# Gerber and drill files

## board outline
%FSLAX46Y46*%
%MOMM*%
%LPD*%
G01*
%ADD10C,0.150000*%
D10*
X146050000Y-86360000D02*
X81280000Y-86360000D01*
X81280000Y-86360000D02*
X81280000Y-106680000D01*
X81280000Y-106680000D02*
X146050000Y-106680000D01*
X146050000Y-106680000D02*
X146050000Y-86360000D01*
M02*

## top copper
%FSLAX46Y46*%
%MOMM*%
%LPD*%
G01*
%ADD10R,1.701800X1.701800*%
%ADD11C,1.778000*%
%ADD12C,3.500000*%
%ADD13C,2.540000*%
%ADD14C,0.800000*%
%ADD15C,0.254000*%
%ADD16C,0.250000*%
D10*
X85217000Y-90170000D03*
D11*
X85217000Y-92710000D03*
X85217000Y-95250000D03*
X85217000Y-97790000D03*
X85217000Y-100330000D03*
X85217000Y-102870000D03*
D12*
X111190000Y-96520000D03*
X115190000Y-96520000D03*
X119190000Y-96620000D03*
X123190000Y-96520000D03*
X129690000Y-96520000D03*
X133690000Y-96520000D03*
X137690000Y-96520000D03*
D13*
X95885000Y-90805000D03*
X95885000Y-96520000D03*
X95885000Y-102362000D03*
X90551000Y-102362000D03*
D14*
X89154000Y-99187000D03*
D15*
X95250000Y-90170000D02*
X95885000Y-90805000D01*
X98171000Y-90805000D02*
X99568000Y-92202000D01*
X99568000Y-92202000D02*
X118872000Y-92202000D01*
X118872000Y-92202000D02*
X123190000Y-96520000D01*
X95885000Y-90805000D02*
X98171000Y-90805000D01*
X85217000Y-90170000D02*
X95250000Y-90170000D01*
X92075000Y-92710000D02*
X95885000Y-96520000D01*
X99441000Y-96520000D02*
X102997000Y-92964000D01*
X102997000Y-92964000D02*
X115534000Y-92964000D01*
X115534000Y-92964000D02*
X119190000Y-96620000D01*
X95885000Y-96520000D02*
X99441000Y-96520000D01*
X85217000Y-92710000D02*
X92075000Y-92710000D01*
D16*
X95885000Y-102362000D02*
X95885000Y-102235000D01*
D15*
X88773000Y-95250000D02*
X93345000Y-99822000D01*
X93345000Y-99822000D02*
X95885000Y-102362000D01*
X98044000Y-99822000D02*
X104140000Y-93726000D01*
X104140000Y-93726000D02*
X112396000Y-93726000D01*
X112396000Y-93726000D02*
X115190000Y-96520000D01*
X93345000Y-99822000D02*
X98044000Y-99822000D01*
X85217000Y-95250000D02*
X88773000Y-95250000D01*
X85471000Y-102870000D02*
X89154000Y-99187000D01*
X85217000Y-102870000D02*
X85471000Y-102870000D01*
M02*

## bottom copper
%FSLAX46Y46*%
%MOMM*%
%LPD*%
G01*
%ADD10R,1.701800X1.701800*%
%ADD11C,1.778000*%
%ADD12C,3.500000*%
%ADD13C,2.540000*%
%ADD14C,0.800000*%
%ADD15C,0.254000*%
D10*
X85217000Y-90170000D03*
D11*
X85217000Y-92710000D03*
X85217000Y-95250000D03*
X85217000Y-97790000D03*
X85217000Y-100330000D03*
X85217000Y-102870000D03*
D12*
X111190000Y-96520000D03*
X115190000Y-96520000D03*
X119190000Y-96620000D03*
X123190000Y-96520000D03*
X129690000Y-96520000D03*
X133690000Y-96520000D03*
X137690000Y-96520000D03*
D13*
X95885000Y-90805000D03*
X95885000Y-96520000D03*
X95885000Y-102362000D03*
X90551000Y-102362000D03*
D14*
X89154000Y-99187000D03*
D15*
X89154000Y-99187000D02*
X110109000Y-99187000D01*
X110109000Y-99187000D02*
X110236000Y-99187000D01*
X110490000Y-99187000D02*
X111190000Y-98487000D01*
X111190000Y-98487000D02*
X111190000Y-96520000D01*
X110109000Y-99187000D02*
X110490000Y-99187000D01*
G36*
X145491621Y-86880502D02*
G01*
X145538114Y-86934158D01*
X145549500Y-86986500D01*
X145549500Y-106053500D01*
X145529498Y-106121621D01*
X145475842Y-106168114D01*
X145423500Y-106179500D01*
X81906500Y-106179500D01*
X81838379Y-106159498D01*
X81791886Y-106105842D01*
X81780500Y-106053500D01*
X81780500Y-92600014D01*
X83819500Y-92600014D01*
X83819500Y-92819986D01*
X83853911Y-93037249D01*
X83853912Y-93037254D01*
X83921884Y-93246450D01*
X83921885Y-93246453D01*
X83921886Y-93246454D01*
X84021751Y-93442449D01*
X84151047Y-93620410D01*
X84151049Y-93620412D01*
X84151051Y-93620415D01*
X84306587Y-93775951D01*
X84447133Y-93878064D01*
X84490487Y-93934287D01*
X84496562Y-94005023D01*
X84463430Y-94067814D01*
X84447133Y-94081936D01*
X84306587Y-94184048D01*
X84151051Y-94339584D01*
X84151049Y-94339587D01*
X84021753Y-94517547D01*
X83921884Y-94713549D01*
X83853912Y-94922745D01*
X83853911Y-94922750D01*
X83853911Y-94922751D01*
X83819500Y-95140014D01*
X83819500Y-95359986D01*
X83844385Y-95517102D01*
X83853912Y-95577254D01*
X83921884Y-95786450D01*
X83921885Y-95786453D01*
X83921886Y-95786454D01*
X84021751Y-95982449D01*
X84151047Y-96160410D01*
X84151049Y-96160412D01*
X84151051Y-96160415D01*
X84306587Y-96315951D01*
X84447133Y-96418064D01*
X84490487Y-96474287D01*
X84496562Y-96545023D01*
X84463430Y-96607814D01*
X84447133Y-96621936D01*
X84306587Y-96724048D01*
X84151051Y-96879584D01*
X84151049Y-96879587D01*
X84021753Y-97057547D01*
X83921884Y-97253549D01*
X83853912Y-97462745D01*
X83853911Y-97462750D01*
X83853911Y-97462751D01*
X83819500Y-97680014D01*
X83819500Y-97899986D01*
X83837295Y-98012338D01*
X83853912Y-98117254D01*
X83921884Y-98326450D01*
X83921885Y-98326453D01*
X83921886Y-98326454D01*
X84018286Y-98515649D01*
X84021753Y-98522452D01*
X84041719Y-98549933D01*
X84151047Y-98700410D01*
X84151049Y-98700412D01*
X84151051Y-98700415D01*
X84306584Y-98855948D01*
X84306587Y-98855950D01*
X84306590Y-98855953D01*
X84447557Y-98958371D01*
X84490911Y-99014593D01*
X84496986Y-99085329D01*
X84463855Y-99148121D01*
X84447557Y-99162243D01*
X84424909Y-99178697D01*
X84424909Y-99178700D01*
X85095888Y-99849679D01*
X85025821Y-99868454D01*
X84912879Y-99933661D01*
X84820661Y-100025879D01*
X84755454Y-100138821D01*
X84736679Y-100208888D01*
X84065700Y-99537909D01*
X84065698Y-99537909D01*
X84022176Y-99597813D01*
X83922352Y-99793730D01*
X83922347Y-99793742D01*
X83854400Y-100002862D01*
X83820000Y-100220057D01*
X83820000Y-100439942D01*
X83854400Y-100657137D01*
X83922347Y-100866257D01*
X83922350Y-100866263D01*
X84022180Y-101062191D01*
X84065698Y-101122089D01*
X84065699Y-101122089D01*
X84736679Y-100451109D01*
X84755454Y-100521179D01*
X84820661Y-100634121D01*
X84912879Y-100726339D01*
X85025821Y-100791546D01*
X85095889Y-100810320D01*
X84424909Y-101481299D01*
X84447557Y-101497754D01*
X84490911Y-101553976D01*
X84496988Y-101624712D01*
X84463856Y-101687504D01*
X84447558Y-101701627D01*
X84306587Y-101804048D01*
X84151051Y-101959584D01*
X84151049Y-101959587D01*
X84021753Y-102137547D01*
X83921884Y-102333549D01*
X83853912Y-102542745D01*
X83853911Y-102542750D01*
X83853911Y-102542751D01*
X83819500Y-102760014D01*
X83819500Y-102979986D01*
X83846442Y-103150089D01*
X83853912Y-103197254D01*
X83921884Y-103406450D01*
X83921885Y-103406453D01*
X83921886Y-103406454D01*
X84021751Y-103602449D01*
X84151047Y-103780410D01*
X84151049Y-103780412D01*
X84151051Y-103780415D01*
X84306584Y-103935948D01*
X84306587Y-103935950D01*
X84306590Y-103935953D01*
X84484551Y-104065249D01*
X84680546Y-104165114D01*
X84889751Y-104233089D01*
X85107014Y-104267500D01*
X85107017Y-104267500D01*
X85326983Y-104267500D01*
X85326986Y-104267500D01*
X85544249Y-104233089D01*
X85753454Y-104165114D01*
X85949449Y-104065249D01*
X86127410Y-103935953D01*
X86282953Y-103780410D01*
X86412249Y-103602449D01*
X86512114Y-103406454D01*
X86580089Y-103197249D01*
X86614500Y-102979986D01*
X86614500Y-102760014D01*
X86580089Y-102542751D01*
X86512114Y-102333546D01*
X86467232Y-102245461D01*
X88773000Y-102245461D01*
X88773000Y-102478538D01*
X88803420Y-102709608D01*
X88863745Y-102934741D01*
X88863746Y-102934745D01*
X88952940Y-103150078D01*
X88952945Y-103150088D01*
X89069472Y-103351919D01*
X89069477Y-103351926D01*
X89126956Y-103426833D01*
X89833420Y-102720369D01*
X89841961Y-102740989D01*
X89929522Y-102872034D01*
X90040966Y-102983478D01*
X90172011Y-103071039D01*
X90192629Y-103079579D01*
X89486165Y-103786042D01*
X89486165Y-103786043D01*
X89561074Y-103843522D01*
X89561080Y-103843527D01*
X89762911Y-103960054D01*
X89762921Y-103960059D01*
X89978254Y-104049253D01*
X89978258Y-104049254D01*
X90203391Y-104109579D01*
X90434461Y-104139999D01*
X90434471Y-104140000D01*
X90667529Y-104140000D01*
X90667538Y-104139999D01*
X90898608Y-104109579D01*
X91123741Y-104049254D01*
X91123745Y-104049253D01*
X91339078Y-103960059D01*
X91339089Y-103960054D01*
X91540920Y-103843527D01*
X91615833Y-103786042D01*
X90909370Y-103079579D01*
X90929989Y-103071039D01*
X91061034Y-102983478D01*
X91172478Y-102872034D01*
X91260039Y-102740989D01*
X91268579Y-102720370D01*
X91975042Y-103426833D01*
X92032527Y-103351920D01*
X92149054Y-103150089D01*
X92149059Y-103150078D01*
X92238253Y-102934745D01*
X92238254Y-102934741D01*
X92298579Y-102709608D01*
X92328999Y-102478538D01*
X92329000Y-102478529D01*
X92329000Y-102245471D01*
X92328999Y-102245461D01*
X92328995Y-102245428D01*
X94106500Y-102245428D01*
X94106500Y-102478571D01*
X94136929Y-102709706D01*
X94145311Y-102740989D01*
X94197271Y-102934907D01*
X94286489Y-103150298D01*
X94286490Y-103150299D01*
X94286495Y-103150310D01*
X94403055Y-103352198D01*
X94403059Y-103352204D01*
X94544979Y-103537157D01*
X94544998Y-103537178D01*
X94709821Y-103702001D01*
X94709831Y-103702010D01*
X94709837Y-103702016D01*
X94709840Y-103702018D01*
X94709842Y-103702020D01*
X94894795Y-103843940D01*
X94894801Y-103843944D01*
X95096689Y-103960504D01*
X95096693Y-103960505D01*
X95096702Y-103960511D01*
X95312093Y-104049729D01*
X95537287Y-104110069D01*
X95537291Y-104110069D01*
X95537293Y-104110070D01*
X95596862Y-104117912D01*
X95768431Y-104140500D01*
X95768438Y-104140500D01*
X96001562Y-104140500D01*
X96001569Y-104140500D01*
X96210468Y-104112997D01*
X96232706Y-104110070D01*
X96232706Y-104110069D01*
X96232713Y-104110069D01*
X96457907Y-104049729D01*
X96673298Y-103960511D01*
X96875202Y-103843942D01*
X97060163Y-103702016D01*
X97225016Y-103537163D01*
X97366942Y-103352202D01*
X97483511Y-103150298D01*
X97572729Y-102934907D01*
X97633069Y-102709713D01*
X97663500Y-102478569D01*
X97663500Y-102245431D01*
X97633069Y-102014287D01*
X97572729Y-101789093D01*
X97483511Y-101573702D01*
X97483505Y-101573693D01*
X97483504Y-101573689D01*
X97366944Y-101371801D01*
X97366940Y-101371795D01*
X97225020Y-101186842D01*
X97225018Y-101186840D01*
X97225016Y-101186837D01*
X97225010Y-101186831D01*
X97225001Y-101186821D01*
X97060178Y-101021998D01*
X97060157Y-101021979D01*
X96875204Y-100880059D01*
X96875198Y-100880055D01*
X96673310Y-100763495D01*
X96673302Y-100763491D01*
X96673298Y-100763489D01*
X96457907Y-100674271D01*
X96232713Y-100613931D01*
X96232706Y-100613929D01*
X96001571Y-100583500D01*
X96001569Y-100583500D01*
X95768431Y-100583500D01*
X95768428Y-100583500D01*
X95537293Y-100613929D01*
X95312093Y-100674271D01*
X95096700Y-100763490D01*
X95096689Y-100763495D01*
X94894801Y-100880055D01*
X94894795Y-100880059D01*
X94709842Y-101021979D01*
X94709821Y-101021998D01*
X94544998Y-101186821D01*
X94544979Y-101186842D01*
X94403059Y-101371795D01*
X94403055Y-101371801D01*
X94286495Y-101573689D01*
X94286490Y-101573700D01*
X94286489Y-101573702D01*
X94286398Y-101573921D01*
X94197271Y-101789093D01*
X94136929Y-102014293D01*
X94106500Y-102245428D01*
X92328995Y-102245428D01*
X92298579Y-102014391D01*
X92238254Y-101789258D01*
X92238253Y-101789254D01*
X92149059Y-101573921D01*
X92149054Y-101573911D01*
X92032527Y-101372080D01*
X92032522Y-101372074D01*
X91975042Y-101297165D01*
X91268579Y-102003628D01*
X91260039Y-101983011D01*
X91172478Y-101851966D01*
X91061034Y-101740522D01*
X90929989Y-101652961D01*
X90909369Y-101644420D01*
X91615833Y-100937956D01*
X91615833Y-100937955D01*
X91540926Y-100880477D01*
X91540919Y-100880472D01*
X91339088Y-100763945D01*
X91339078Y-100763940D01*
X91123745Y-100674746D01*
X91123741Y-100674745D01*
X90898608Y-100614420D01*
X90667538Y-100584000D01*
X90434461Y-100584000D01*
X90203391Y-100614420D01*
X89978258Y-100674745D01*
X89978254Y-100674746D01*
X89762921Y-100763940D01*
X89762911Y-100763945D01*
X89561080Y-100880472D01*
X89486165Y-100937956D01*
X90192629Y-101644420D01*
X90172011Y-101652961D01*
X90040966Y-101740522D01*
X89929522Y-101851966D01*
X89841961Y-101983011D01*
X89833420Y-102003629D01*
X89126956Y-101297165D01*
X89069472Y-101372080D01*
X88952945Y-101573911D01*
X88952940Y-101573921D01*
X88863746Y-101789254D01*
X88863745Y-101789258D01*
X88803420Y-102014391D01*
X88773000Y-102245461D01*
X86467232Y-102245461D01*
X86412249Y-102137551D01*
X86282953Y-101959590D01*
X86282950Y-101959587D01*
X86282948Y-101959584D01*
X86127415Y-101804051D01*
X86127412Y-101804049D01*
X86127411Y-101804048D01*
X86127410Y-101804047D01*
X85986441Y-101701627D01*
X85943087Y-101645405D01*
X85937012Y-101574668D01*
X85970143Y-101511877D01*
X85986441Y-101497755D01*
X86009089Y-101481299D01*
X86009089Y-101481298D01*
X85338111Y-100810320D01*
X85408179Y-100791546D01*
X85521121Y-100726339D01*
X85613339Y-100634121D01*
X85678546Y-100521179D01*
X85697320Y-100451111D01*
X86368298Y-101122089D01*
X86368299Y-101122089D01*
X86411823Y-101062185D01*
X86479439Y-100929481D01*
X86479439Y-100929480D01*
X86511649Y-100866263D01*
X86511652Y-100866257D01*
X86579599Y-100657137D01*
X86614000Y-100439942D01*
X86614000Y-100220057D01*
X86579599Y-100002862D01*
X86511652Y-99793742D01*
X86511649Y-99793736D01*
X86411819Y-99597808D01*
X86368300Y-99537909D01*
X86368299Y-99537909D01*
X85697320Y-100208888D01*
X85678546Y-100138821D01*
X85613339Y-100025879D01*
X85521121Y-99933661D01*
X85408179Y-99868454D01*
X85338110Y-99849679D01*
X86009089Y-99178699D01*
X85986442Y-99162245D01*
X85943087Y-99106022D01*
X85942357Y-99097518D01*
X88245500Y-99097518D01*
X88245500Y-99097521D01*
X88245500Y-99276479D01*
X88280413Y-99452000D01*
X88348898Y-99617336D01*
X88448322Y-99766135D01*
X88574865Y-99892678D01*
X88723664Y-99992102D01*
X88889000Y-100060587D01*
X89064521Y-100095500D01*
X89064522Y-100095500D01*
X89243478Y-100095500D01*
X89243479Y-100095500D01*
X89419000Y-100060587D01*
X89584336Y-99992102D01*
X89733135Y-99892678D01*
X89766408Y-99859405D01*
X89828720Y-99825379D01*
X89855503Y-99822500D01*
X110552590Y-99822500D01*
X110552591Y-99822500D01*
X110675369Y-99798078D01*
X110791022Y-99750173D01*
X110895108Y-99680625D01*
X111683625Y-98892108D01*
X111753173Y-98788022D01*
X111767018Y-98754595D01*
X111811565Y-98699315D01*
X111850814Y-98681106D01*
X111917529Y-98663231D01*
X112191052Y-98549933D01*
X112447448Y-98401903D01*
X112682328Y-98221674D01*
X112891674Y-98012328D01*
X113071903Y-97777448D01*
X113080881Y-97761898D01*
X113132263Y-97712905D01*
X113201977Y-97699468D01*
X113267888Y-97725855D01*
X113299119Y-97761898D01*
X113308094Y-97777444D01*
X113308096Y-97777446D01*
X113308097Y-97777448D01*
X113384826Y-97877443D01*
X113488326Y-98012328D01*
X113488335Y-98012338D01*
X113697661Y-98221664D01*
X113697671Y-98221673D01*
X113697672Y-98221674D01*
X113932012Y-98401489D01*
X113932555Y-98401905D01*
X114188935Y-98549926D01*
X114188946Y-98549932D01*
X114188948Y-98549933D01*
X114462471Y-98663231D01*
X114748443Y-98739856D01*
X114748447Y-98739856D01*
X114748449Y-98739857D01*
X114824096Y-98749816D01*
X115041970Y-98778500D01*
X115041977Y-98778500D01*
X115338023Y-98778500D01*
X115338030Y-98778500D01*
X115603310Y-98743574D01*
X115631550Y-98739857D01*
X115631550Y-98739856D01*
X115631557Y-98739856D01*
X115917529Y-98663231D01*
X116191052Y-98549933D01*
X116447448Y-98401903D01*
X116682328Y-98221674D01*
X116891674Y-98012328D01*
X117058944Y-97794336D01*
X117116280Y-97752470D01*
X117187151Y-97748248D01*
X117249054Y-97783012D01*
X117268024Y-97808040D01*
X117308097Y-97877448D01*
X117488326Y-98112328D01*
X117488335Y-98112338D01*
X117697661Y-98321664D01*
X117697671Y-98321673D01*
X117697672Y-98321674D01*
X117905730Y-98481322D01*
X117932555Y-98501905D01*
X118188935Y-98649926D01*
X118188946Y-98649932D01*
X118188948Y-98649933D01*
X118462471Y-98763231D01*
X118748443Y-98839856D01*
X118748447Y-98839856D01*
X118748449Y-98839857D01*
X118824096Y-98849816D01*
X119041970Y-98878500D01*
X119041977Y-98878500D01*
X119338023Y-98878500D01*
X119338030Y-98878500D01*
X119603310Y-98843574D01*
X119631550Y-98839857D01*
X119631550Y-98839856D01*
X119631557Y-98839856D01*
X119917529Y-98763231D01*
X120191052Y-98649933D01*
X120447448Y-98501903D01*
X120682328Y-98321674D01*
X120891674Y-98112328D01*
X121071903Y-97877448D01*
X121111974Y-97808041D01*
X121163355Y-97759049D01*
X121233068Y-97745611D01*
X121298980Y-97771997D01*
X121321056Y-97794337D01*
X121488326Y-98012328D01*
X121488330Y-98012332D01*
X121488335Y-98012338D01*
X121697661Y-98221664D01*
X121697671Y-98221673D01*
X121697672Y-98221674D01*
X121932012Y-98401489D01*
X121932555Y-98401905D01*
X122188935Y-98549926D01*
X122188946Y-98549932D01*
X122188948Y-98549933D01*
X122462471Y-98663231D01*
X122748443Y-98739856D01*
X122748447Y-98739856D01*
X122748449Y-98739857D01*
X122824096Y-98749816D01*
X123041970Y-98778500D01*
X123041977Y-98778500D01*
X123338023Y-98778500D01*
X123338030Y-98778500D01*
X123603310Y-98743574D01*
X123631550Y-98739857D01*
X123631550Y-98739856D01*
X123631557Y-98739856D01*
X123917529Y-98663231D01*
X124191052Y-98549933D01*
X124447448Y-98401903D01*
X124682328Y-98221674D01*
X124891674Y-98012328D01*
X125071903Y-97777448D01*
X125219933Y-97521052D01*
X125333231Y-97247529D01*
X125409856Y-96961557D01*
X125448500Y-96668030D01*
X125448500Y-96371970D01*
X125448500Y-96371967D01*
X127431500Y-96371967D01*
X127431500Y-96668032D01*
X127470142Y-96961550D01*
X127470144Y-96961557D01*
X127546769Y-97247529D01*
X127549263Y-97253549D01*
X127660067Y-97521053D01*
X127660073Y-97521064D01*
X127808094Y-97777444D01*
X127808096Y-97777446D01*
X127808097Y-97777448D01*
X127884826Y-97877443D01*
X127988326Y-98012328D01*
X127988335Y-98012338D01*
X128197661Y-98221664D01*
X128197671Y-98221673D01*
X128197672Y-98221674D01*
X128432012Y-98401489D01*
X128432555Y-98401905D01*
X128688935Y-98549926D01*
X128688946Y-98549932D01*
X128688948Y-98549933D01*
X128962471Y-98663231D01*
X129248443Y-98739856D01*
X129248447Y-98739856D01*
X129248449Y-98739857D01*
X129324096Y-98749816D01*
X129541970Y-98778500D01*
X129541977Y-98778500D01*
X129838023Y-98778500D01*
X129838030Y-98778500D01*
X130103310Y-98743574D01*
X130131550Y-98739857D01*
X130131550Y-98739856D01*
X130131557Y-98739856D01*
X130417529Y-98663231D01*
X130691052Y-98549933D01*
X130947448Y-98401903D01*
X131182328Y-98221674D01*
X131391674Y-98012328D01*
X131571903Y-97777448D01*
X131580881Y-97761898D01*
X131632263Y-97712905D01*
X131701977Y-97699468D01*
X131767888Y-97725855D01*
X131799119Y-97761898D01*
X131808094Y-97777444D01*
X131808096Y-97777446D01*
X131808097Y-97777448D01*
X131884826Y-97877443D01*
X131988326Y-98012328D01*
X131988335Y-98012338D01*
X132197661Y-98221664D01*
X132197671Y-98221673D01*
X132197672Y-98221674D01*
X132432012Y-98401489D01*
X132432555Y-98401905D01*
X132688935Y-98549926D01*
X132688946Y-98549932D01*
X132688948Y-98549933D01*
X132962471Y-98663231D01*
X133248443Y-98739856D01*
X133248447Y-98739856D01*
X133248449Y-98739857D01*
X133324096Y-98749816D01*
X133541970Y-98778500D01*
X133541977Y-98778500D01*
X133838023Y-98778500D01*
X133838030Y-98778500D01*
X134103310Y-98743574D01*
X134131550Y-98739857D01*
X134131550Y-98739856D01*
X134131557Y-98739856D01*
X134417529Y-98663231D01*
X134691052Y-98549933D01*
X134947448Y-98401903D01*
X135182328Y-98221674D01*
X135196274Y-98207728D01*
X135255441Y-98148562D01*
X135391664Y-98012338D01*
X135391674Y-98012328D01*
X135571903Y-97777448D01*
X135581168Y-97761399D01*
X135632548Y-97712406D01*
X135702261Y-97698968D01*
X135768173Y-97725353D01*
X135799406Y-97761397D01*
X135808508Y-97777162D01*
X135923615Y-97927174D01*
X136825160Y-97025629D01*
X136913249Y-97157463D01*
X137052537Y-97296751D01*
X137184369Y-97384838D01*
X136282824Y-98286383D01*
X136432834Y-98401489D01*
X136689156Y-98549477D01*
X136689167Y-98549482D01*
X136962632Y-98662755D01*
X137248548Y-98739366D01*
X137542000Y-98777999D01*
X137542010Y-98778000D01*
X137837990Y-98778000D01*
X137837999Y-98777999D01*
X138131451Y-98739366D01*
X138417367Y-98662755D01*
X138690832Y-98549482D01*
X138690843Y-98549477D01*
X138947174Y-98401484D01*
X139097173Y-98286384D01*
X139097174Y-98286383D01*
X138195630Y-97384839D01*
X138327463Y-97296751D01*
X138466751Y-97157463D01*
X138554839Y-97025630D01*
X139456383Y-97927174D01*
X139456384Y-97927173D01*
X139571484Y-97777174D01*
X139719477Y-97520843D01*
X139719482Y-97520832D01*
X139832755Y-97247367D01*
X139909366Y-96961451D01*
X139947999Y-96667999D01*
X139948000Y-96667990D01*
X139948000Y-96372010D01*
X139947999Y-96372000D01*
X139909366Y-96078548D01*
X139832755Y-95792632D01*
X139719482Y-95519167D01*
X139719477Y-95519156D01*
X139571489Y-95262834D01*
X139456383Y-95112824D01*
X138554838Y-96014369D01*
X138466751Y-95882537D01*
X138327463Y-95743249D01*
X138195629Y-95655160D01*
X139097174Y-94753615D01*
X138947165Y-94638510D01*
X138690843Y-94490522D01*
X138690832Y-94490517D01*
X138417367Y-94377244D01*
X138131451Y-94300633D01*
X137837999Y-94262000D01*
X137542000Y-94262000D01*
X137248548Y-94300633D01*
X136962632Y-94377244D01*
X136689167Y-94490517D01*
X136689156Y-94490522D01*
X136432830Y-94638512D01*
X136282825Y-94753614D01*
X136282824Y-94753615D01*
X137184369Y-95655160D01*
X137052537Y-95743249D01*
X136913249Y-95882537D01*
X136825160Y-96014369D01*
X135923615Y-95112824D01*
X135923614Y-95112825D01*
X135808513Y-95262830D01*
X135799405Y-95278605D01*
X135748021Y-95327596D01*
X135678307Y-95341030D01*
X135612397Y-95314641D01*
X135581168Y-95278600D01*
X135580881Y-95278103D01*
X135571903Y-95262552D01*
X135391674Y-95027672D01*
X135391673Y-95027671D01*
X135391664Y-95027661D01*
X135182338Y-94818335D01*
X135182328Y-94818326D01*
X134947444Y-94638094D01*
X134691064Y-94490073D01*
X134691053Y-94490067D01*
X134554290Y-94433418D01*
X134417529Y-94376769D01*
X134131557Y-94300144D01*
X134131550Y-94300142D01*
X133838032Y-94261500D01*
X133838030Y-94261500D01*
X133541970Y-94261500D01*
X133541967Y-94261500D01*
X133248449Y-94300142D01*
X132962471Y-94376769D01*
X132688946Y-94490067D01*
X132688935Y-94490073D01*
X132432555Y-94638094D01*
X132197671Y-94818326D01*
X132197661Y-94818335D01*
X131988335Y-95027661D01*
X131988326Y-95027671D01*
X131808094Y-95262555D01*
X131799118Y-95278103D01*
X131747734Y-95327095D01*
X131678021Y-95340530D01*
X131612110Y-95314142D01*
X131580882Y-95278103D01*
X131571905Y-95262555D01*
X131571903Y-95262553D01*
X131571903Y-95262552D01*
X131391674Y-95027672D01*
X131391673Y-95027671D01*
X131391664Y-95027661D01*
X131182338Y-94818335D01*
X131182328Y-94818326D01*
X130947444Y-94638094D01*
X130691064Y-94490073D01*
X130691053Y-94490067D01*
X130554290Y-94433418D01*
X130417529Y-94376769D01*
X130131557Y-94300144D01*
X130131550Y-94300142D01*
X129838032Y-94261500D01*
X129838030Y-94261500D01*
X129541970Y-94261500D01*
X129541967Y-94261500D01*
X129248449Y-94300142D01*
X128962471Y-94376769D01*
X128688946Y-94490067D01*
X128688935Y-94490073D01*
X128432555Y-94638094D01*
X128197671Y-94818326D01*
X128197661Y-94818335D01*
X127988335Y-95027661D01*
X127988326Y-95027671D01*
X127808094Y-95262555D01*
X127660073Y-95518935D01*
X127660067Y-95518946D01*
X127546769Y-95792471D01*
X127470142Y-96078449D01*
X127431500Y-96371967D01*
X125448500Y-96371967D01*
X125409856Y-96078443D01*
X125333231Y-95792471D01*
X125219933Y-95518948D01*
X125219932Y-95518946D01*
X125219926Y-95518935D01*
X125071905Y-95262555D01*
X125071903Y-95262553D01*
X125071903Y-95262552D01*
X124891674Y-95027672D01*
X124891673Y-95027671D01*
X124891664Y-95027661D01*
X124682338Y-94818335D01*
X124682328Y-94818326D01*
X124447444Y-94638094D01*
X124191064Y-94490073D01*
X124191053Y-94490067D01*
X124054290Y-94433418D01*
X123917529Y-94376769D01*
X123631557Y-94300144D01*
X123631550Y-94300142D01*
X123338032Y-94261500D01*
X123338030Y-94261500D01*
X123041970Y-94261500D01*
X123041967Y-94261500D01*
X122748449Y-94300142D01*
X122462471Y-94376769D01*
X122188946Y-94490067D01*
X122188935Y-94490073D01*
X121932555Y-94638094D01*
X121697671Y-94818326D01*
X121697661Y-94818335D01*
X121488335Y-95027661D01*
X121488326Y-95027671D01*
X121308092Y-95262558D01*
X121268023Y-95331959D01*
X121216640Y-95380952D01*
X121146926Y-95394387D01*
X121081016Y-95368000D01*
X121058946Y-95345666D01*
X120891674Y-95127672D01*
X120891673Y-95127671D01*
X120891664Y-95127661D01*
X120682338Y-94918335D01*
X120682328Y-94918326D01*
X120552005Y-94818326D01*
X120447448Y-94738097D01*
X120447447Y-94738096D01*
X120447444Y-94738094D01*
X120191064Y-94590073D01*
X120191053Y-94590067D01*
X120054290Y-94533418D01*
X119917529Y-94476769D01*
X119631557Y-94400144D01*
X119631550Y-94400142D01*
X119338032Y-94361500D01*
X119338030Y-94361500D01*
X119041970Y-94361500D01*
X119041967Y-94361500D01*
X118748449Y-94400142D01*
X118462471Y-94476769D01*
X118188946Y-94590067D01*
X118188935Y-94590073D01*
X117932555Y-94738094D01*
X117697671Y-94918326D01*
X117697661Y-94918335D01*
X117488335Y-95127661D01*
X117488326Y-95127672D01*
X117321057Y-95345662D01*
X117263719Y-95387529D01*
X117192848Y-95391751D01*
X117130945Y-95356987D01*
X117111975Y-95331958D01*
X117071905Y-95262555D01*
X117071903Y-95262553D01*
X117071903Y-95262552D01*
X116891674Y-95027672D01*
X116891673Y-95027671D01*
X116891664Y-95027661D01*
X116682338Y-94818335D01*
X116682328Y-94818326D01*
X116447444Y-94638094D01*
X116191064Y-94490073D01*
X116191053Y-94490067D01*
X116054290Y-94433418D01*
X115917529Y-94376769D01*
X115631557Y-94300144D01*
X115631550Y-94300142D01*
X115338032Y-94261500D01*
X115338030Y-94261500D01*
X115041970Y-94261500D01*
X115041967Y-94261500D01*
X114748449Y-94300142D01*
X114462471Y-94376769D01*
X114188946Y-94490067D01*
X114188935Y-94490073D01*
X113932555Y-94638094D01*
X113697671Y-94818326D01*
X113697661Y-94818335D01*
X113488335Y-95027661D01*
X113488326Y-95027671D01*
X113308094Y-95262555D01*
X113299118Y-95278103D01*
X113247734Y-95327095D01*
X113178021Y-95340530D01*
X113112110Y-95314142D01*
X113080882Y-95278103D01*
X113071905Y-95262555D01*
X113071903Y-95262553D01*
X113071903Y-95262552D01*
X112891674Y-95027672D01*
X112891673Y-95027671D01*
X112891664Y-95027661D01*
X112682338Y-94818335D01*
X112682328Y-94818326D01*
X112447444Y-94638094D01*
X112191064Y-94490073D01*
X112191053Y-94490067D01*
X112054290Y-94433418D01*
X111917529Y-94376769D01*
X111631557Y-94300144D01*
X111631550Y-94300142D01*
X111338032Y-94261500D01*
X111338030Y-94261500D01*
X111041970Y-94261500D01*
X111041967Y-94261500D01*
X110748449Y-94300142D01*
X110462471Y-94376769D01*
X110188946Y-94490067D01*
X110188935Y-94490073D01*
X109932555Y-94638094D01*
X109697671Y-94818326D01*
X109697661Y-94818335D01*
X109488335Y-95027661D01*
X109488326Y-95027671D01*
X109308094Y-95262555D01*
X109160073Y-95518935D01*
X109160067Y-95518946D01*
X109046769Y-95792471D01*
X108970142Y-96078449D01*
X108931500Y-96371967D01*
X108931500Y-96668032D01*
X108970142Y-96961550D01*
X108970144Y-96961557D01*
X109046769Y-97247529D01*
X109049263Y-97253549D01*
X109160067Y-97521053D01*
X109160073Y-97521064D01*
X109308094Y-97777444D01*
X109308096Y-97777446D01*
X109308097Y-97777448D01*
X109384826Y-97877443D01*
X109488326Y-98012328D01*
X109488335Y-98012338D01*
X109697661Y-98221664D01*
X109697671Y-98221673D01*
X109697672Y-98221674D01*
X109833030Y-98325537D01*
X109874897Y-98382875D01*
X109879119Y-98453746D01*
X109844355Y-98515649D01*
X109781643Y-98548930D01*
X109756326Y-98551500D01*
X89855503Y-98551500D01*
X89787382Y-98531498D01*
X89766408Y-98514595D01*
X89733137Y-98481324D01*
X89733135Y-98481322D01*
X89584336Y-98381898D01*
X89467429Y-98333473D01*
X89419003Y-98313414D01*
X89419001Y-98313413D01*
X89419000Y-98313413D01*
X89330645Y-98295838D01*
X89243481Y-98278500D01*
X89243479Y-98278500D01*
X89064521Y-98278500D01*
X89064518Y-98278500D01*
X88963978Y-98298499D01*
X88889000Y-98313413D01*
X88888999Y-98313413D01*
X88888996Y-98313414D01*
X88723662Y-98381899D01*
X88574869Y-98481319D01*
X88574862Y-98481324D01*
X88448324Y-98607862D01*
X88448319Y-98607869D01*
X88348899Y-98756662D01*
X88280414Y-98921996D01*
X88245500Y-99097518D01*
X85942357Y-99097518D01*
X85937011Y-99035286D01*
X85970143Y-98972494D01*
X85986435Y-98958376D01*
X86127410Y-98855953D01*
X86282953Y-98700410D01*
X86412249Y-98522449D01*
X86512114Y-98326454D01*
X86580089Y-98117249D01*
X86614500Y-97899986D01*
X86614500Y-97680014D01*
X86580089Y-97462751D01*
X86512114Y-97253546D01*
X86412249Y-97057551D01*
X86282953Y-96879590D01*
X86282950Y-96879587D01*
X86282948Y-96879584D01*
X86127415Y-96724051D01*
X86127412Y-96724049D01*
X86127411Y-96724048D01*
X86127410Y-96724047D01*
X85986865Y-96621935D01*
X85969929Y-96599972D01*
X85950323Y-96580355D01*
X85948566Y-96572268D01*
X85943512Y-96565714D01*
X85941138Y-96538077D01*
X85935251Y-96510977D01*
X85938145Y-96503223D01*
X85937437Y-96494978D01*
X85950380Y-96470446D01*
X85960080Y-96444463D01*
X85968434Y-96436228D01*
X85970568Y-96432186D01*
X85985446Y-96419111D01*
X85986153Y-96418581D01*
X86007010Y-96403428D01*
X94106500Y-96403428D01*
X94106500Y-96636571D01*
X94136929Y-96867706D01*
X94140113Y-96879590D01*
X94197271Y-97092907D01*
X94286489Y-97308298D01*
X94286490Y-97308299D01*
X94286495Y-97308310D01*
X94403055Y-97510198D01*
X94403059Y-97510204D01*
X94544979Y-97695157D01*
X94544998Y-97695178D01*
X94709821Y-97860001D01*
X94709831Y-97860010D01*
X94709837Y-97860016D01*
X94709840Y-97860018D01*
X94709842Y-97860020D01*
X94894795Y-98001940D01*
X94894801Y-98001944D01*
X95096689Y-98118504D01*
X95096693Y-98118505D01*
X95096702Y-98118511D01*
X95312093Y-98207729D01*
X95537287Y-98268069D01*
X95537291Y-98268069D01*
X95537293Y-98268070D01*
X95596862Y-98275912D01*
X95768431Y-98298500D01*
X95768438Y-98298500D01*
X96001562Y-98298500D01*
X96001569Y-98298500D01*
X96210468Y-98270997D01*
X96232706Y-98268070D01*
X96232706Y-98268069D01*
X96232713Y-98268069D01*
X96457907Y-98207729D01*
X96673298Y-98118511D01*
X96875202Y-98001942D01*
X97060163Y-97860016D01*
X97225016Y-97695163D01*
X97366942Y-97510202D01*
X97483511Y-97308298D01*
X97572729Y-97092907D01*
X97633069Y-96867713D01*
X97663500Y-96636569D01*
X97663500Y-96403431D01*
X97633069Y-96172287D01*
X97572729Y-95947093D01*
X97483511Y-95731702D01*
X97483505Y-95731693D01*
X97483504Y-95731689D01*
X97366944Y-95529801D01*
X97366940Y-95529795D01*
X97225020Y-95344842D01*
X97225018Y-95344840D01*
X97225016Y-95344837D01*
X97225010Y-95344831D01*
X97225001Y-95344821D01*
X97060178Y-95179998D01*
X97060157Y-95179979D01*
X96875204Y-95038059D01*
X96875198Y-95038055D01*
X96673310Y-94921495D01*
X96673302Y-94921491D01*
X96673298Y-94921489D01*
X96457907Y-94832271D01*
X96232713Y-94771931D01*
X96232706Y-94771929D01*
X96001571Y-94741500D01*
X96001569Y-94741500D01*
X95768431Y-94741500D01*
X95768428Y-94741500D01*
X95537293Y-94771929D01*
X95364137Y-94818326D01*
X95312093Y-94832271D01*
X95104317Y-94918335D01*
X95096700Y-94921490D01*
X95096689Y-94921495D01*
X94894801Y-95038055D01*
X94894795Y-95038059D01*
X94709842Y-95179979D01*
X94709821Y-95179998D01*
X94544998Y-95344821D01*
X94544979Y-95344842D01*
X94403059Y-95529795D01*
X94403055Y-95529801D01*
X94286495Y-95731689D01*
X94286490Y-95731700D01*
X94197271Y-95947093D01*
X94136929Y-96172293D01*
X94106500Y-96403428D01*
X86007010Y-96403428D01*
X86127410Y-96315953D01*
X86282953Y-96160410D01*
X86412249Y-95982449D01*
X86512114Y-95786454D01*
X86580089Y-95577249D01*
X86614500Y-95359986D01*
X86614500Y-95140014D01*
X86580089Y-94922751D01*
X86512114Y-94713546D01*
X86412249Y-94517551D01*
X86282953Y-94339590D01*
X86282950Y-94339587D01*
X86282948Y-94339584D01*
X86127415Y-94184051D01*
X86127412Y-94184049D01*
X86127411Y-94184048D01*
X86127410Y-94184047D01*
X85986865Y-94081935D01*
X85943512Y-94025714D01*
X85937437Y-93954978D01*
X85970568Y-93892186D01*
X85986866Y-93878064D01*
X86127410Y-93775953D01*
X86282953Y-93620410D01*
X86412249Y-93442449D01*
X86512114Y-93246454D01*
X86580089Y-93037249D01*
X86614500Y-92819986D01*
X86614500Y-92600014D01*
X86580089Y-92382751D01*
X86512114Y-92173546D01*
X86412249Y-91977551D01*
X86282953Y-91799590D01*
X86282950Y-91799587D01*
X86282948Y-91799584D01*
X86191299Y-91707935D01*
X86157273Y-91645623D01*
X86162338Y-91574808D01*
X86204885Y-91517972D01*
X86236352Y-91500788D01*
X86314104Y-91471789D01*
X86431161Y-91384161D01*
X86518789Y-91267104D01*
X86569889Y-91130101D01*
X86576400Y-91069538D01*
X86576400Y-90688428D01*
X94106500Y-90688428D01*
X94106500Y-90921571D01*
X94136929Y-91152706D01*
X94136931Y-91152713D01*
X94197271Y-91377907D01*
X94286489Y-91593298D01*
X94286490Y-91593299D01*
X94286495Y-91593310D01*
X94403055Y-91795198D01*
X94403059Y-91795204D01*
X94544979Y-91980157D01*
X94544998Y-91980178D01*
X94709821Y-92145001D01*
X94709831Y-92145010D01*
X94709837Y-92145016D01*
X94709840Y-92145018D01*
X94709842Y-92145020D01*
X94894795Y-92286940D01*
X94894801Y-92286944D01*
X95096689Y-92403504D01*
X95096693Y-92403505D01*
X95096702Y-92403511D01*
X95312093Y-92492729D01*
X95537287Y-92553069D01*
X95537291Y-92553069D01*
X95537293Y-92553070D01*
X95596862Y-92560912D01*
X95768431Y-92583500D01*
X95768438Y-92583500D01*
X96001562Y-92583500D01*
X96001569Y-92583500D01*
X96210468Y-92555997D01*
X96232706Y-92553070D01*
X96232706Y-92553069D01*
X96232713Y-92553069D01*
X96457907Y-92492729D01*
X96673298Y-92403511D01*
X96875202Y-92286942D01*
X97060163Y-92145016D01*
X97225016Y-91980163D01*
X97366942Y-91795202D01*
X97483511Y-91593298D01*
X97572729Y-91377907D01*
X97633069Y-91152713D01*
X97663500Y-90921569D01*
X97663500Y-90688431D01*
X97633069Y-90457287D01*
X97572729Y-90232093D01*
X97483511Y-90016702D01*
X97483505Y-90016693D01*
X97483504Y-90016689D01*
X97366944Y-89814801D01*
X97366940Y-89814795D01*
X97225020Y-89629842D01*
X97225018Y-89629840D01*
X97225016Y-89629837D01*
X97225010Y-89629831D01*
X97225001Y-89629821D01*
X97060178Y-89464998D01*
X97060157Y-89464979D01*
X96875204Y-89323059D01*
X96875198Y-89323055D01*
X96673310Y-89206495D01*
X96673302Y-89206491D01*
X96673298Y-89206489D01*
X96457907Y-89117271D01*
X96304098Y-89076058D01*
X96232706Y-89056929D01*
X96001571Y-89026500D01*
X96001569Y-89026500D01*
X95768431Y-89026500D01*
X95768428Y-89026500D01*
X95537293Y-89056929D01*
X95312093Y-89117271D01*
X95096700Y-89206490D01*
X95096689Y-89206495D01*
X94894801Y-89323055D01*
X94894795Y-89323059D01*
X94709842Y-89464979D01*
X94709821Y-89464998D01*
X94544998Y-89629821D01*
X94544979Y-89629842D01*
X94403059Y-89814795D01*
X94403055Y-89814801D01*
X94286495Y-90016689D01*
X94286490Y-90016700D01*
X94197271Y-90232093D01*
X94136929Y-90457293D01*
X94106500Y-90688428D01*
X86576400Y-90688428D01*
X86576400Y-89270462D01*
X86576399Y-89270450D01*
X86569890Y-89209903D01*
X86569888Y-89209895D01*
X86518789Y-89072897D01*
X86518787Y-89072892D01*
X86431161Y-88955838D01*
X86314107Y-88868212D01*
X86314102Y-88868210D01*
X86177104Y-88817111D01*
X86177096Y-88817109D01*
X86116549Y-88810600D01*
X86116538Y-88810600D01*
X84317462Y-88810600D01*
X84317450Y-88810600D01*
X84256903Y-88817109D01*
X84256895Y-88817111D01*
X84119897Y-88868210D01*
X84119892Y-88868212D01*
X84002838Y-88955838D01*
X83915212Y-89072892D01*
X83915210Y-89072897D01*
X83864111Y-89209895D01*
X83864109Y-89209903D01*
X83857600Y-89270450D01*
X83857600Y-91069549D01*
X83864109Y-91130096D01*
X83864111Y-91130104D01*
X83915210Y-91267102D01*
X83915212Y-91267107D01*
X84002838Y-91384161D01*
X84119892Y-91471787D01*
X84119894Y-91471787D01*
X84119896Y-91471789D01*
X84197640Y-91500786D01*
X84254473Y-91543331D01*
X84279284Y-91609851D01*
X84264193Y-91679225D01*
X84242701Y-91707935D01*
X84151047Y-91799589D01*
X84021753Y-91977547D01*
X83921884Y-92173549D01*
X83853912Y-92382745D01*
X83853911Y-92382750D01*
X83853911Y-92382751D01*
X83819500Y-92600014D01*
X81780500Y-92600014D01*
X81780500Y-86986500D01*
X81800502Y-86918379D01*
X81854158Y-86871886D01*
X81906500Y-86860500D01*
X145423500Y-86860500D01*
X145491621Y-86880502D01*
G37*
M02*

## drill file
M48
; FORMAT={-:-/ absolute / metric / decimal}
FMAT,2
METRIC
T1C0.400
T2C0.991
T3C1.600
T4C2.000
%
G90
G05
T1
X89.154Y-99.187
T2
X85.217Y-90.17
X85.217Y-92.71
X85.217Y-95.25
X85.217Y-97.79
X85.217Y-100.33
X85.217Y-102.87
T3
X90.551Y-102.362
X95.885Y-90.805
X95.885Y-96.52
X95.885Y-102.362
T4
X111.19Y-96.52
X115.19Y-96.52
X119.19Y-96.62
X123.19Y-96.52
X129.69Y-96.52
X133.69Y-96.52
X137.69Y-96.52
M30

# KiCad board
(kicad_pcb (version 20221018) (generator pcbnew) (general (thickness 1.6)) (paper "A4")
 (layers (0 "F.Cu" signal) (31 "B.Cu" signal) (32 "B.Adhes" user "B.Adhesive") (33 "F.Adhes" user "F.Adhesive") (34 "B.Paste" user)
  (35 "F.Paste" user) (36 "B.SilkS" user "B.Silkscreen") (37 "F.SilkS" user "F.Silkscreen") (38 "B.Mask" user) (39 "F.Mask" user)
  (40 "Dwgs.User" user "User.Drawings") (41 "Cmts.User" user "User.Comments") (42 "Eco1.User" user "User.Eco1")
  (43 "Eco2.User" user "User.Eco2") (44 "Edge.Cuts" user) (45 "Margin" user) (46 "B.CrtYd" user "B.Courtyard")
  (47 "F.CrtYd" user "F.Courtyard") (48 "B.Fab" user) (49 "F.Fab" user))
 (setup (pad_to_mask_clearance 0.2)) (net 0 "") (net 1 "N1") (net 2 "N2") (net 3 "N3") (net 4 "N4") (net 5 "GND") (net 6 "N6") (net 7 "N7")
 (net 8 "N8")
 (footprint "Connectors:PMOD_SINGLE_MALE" (layer "F.Cu") (at 83.185 96.52 90)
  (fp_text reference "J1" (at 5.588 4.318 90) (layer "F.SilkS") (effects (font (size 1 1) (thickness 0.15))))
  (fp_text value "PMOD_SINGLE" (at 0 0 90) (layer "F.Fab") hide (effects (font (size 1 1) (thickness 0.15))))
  (pad "1" thru_hole rect (at 6.35 2.032 270) (size 1.7018 1.7018) (drill 0.9906) (layers "*.Cu" "*.Mask" "F.SilkS") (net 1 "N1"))
  (pad "2" thru_hole circle (at 3.81 2.032 270) (size 1.778 1.778) (drill 0.9906) (layers "*.Cu" "*.Mask" "F.SilkS") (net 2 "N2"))
  (pad "3" thru_hole circle (at 1.27 2.032 270) (size 1.778 1.778) (drill 0.9906) (layers "*.Cu" "*.Mask" "F.SilkS") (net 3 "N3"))
  (pad "4" thru_hole circle (at -1.27 2.032 270) (size 1.778 1.778) (drill 0.9906) (layers "*.Cu" "*.Mask" "F.SilkS") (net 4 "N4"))
  (pad "5" thru_hole circle (at -3.81 2.032 270) (size 1.778 1.778) (drill 0.9906) (layers "*.Cu" "*.Mask" "F.SilkS") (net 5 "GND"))
  (pad "6" thru_hole circle (at -6.35 2.032 270) (size 1.778 1.778) (drill 0.9906) (layers "*.Cu" "*.Mask" "F.SilkS") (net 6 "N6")))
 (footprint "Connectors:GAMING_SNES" (layer "F.Cu") (at 123.19 96.52)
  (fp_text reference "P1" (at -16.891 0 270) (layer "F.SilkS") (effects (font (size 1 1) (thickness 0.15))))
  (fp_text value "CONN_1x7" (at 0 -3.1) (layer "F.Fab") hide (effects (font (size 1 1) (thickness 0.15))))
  (pad "1" thru_hole circle (at -12 0) (size 3.5 3.5) (drill 2) (layers "*.Cu" "*.Mask" "F.SilkS") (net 6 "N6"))
  (pad "2" thru_hole circle (at -8 0) (size 3.5 3.5) (drill 2) (layers "*.Cu" "*.Mask" "F.SilkS") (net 3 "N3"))
  (pad "3" thru_hole circle (at -4 0.1) (size 3.5 3.5) (drill 2) (layers "*.Cu" "*.Mask" "F.SilkS") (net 2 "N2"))
  (pad "4" thru_hole circle (at 0 0) (size 3.5 3.5) (drill 2) (layers "*.Cu" "*.Mask" "F.SilkS") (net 1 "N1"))
  (pad "5" thru_hole circle (at 6.5 0) (size 3.5 3.5) (drill 2) (layers "*.Cu" "*.Mask" "F.SilkS") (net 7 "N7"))
  (pad "6" thru_hole circle (at 10.5 0) (size 3.5 3.5) (drill 2) (layers "*.Cu" "*.Mask" "F.SilkS") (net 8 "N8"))
  (pad "7" thru_hole circle (at 14.5 0) (size 3.5 3.5) (drill 2) (layers "*.Cu" "*.Mask" "F.SilkS") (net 5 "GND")))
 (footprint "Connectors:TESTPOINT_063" (layer "F.Cu") (at 95.885 90.805)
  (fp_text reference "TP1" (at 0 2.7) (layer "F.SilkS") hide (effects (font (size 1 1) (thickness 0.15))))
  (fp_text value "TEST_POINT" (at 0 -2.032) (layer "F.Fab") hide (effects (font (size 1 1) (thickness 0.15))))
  (pad "1" thru_hole circle (at 0 0) (size 2.54 2.54) (drill 1.6002) (layers "*.Cu" "*.Mask" "F.SilkS") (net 1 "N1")))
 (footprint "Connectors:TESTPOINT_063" (layer "F.Cu") (at 95.885 96.52)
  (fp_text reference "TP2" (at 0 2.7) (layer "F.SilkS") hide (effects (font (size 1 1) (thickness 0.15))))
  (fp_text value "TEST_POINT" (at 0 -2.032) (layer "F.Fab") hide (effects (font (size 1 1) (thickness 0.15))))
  (pad "1" thru_hole circle (at 0 0) (size 2.54 2.54) (drill 1.6002) (layers "*.Cu" "*.Mask" "F.SilkS") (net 2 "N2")))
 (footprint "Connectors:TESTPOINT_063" (layer "F.Cu") (at 95.885 102.362)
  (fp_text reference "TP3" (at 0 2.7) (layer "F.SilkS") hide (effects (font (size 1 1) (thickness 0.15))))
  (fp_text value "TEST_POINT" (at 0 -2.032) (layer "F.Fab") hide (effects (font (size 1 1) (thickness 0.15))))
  (pad "1" thru_hole circle (at 0 0) (size 2.54 2.54) (drill 1.6002) (layers "*.Cu" "*.Mask" "F.SilkS") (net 3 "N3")))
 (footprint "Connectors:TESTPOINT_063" (layer "F.Cu") (at 90.551 102.362)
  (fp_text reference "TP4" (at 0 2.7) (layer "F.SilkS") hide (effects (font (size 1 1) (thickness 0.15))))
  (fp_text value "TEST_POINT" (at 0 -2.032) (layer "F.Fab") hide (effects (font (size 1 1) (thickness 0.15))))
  (pad "1" thru_hole circle (at 0 0) (size 2.54 2.54) (drill 1.6002) (layers "*.Cu" "*.Mask" "F.SilkS") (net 5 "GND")))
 (gr_line (start 146.05 86.36) (end 81.28 86.36) (stroke (width 0.15) (type solid)) (layer "Edge.Cuts"))
 (gr_line (start 81.28 86.36) (end 81.28 106.68) (stroke (width 0.15) (type solid)) (layer "Edge.Cuts"))
 (gr_line (start 81.28 106.68) (end 146.05 106.68) (stroke (width 0.15) (type solid)) (layer "Edge.Cuts"))
 (gr_line (start 146.05 106.68) (end 146.05 86.36) (stroke (width 0.15) (type solid)) (layer "Edge.Cuts"))
 (segment (start 95.25 90.17) (end 95.885 90.805) (width 0.254) (layer "F.Cu") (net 1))
 (segment (start 98.171 90.805) (end 99.568 92.202) (width 0.254) (layer "F.Cu") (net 1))
 (segment (start 99.568 92.202) (end 118.872 92.202) (width 0.254) (layer "F.Cu") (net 1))
 (segment (start 118.872 92.202) (end 123.19 96.52) (width 0.254) (layer "F.Cu") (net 1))
 (segment (start 95.885 90.805) (end 98.171 90.805) (width 0.254) (layer "F.Cu") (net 1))
 (segment (start 85.217 90.17) (end 95.25 90.17) (width 0.254) (layer "F.Cu") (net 1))
 (segment (start 92.075 92.71) (end 95.885 96.52) (width 0.254) (layer "F.Cu") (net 2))
 (segment (start 99.441 96.52) (end 102.997 92.964) (width 0.254) (layer "F.Cu") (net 2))
 (segment (start 102.997 92.964) (end 115.534 92.964) (width 0.254) (layer "F.Cu") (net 2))
 (segment (start 115.534 92.964) (end 119.19 96.62) (width 0.254) (layer "F.Cu") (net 2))
 (segment (start 95.885 96.52) (end 99.441 96.52) (width 0.254) (layer "F.Cu") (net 2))
 (segment (start 85.217 92.71) (end 92.075 92.71) (width 0.254) (layer "F.Cu") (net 2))
 (segment (start 95.885 102.362) (end 95.885 102.235) (width 0.25) (layer "F.Cu") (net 3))
 (segment (start 88.773 95.25) (end 93.345 99.822) (width 0.254) (layer "F.Cu") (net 3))
 (segment (start 93.345 99.822) (end 95.885 102.362) (width 0.254) (layer "F.Cu") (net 3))
 (segment (start 98.044 99.822) (end 104.14 93.726) (width 0.254) (layer "F.Cu") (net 3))
 (segment (start 104.14 93.726) (end 112.396 93.726) (width 0.254) (layer "F.Cu") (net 3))
 (segment (start 112.396 93.726) (end 115.19 96.52) (width 0.254) (layer "F.Cu") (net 3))
 (segment (start 93.345 99.822) (end 98.044 99.822) (width 0.254) (layer "F.Cu") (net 3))
 (segment (start 85.217 95.25) (end 88.773 95.25) (width 0.254) (layer "F.Cu") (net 3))
 (segment (start 85.471 102.87) (end 89.154 99.187) (width 0.254) (layer "F.Cu") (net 6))
 (segment (start 85.217 102.87) (end 85.471 102.87) (width 0.254) (layer "F.Cu") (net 6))
 (via (at 89.154 99.187) (size 0.8) (drill 0.4) (layers "F.Cu" "B.Cu") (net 6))
 (segment (start 89.154 99.187) (end 110.109 99.187) (width 0.254) (layer "B.Cu") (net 6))
 (segment (start 110.109 99.187) (end 110.236 99.187) (width 0.254) (layer "B.Cu") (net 6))
 (segment (start 110.49 99.187) (end 111.19 98.487) (width 0.254) (layer "B.Cu") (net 6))
 (segment (start 111.19 98.487) (end 111.19 96.52) (width 0.254) (layer "B.Cu") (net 6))
 (segment (start 110.109 99.187) (end 110.49 99.187) (width 0.254) (layer "B.Cu") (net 6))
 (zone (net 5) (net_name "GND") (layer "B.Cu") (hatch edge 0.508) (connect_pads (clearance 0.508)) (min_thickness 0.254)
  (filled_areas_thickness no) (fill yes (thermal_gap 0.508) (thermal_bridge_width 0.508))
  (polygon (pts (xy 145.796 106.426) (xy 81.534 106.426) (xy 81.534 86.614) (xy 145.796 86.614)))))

